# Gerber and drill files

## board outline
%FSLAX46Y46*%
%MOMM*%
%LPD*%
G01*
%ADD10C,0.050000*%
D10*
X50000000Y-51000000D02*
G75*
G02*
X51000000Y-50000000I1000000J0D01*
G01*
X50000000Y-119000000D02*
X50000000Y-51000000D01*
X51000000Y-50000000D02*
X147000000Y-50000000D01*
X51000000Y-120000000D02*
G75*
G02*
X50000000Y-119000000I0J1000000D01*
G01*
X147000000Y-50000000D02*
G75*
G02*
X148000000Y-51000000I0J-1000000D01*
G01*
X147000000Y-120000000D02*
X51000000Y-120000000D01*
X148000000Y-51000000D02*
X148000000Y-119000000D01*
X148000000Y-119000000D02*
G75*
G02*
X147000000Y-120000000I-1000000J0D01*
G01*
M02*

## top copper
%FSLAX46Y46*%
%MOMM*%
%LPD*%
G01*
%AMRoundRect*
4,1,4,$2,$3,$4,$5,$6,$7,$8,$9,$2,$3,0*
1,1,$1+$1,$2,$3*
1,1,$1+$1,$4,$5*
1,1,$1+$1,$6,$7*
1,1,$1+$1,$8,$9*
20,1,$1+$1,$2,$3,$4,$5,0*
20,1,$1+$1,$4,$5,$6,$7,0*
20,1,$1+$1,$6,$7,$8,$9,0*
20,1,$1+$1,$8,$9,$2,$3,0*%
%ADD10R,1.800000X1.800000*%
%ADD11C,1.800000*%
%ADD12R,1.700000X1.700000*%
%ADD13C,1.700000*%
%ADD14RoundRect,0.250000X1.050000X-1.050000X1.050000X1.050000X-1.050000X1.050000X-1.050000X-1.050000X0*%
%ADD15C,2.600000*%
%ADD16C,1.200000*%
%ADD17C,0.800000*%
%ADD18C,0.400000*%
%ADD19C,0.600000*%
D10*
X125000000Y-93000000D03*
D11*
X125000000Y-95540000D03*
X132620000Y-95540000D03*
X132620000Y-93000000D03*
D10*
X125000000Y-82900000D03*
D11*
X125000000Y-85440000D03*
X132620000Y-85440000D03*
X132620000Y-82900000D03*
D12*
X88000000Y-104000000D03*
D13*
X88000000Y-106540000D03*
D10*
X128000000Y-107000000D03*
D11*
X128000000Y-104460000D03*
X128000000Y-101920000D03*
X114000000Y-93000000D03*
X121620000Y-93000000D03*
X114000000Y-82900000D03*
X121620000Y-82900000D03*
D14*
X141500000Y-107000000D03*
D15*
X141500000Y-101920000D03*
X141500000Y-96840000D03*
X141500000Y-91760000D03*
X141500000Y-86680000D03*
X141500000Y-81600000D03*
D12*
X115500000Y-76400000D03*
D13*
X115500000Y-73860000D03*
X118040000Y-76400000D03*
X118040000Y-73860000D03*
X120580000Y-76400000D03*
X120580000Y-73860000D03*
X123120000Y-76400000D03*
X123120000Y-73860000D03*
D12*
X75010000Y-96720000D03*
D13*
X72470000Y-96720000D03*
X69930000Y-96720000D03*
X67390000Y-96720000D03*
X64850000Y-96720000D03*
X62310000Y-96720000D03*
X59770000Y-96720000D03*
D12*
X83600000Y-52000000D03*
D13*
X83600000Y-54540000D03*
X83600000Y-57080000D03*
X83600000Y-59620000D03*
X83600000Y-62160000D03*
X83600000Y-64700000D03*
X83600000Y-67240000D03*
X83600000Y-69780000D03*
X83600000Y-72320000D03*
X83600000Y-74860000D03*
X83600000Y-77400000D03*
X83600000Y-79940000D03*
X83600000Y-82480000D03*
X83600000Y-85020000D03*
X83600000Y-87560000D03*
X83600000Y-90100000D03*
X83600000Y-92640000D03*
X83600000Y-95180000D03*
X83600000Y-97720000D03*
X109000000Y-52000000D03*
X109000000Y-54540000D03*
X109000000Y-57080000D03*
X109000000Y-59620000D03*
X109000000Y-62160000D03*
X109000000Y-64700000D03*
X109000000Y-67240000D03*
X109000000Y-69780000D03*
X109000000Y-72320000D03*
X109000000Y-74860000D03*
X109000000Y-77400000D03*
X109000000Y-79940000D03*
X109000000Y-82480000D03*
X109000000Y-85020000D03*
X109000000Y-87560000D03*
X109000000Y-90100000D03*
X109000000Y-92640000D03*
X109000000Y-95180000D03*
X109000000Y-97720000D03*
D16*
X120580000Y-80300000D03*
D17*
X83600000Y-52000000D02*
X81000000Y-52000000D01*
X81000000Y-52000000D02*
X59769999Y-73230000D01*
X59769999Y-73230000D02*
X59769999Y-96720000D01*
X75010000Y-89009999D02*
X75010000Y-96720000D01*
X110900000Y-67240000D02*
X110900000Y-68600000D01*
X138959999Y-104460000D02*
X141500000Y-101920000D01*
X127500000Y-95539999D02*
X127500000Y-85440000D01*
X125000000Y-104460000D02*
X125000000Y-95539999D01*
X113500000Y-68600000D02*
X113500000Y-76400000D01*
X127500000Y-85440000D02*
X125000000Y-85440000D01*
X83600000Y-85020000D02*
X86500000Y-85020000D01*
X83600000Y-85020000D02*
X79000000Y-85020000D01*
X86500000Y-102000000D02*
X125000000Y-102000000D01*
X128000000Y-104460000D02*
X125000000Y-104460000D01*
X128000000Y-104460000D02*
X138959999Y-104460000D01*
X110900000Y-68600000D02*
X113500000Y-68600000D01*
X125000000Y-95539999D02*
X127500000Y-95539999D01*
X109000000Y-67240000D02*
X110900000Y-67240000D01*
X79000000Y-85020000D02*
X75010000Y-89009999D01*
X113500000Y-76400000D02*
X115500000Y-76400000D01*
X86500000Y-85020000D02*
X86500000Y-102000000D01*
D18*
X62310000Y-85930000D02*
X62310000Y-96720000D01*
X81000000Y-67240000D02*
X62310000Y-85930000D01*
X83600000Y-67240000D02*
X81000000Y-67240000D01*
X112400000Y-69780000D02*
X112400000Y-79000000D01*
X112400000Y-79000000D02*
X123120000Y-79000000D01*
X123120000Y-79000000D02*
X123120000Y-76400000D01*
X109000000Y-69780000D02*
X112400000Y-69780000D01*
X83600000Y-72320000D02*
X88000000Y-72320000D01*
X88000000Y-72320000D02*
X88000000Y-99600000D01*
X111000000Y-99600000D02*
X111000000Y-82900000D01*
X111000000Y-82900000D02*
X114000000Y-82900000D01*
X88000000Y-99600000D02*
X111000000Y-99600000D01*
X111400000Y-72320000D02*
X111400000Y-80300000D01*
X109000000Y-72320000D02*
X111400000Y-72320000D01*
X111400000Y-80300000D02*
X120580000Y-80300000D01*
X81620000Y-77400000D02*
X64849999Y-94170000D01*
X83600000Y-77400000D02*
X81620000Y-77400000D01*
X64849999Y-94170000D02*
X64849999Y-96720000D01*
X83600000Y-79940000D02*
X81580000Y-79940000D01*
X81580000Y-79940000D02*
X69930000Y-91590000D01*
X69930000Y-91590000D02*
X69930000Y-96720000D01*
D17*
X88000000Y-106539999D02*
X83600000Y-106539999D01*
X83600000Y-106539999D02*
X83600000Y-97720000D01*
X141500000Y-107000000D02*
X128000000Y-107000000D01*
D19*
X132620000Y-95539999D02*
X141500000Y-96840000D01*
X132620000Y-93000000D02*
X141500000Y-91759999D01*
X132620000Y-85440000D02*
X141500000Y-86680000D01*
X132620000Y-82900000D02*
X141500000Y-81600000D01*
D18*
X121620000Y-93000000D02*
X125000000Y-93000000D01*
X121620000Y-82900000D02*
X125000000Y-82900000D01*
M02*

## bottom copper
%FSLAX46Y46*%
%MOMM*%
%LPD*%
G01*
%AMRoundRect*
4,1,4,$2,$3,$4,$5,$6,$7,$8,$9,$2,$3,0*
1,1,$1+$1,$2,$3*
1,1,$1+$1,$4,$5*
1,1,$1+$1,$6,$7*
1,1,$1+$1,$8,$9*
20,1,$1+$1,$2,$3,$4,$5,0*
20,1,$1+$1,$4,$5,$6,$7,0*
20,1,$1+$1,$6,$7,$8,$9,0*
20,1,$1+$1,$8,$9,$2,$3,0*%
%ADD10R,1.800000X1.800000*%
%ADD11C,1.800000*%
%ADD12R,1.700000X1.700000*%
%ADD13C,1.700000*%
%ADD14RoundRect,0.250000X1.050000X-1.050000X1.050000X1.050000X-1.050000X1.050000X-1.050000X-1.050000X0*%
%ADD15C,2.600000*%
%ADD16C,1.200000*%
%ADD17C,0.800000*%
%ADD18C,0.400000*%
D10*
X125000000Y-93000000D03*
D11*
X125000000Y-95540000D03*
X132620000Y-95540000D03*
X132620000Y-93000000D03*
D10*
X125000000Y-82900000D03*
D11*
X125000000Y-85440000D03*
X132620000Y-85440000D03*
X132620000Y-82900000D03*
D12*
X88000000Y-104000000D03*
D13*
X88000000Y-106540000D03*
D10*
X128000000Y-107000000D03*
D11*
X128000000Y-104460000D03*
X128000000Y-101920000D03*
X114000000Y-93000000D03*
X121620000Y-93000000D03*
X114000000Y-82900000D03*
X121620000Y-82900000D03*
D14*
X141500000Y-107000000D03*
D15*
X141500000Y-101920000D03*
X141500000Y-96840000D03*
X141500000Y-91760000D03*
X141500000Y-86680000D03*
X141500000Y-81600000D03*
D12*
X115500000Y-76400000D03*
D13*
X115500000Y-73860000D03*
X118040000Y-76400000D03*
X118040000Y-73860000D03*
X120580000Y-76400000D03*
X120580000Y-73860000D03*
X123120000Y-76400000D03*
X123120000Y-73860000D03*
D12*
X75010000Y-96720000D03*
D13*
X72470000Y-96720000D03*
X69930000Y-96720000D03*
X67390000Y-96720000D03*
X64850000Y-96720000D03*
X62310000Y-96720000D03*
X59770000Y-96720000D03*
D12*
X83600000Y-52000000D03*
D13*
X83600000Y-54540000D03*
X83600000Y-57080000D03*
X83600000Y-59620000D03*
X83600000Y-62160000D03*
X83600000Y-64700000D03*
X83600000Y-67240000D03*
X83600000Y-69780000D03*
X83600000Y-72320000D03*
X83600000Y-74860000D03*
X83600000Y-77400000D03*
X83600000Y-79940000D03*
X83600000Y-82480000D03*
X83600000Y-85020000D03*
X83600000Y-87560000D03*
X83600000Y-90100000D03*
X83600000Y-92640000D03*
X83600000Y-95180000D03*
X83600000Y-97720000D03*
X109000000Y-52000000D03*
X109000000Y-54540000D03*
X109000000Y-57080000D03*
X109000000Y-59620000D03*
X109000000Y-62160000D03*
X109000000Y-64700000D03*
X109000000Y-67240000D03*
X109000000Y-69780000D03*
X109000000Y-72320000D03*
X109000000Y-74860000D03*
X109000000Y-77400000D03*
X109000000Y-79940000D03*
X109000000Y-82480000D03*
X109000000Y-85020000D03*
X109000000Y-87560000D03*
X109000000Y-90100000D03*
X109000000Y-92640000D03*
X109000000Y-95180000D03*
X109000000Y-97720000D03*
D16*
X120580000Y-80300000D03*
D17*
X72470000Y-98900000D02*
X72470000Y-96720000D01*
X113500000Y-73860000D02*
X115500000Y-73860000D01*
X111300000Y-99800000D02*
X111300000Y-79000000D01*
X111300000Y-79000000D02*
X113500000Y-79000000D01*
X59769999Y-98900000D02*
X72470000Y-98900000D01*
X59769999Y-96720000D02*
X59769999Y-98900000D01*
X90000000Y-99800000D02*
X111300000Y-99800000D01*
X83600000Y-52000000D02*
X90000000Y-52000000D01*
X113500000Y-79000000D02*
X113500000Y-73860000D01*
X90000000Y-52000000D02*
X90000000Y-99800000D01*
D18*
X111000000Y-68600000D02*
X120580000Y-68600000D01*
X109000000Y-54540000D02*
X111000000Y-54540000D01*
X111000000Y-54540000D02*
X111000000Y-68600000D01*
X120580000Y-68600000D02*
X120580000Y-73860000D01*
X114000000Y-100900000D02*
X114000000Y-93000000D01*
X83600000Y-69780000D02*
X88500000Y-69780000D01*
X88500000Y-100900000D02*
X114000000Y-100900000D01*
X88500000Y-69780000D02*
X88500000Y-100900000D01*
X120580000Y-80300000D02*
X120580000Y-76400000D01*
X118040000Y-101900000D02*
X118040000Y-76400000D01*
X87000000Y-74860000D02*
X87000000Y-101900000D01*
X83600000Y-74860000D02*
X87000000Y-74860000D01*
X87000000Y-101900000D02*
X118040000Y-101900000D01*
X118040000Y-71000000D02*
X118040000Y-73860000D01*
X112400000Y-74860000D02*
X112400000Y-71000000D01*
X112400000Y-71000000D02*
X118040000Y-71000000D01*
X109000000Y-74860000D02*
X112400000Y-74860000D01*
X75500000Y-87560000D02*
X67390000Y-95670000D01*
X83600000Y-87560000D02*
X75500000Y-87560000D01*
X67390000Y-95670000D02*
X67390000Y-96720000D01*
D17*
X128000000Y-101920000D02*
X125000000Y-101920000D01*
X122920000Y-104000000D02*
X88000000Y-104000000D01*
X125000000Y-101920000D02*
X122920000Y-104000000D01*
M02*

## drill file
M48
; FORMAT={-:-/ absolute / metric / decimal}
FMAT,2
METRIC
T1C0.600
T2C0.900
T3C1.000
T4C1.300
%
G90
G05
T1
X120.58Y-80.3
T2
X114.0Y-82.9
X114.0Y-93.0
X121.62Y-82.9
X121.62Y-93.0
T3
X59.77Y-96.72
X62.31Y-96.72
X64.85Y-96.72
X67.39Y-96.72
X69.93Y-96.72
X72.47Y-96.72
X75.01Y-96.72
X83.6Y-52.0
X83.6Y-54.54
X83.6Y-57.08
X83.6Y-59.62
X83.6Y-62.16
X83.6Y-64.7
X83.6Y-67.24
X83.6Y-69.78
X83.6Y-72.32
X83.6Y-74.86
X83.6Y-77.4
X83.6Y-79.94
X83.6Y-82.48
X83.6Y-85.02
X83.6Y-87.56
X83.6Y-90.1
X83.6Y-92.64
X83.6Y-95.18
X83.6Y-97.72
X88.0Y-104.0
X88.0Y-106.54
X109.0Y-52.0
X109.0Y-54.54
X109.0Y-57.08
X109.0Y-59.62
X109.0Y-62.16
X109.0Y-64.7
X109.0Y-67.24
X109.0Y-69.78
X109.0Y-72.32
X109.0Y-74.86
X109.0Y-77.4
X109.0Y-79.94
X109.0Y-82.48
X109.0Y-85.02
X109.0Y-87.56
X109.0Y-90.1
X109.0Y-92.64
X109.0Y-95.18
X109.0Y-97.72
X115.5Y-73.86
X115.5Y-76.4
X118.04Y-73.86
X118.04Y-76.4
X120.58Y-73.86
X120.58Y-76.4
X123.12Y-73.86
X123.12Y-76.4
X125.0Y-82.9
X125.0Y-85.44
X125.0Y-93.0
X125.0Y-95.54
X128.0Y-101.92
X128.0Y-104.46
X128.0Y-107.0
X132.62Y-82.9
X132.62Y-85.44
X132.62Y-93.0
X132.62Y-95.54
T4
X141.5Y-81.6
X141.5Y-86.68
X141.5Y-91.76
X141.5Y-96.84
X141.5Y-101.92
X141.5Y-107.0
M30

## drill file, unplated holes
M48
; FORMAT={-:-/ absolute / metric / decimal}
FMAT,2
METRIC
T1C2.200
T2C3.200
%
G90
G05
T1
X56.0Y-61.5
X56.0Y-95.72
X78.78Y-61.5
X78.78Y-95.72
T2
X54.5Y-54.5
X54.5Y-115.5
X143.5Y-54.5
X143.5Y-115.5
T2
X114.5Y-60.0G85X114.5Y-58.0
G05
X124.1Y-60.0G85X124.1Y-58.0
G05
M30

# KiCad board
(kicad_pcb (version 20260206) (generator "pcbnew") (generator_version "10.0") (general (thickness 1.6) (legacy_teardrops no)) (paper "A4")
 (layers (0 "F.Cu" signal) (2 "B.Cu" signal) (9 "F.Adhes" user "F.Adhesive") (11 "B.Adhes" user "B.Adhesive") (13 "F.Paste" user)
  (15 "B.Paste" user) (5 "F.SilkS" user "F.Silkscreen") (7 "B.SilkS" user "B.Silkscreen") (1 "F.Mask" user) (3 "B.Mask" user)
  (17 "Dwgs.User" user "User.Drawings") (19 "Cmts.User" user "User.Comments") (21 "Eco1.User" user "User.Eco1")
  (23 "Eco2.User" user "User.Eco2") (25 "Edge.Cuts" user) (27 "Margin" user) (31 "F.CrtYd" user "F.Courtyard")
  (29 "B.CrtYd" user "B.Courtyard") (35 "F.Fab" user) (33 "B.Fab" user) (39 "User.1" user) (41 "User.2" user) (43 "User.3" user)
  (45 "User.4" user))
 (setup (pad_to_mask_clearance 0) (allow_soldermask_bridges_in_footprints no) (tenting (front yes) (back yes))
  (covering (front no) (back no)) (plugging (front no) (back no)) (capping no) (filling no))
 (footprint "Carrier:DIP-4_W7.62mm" (layer "F.Cu") (at 125 93)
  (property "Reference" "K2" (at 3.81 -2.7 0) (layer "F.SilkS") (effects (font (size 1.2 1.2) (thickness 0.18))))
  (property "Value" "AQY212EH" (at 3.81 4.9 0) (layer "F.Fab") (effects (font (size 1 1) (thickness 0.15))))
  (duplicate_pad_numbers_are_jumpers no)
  (pad "1" thru_hole rect (at 0 0) (size 1.8 1.8) (drill 1) (layers "*.Cu" "*.Mask") (remove_unused_layers no) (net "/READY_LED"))
  (pad "2" thru_hole circle (at 0 2.54) (size 1.8 1.8) (drill 1) (layers "*.Cu" "*.Mask") (remove_unused_layers no) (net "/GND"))
  (pad "3" thru_hole circle (at 7.62 2.54) (size 1.8 1.8) (drill 1) (layers "*.Cu" "*.Mask") (remove_unused_layers no) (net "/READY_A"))
  (pad "4" thru_hole circle (at 7.62 0) (size 1.8 1.8) (drill 1) (layers "*.Cu" "*.Mask") (remove_unused_layers no) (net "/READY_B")))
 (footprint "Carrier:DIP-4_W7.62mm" (layer "F.Cu") (at 125 82.9)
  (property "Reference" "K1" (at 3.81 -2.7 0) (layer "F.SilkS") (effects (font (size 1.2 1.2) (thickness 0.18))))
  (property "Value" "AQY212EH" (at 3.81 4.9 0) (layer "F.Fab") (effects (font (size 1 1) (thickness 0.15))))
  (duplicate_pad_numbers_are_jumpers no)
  (pad "1" thru_hole rect (at 0 0) (size 1.8 1.8) (drill 1) (layers "*.Cu" "*.Mask") (remove_unused_layers no) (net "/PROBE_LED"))
  (pad "2" thru_hole circle (at 0 2.54) (size 1.8 1.8) (drill 1) (layers "*.Cu" "*.Mask") (remove_unused_layers no) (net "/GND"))
  (pad "3" thru_hole circle (at 7.62 2.54) (size 1.8 1.8) (drill 1) (layers "*.Cu" "*.Mask") (remove_unused_layers no) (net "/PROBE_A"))
  (pad "4" thru_hole circle (at 7.62 0) (size 1.8 1.8) (drill 1) (layers "*.Cu" "*.Mask") (remove_unused_layers no) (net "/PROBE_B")))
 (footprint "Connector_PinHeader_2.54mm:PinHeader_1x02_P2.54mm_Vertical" (layer "F.Cu") (at 88 104)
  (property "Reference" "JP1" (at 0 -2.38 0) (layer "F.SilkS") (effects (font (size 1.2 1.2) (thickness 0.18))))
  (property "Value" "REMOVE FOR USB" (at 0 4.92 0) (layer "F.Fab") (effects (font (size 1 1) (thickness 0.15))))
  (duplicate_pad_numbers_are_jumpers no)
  (pad "1" thru_hole rect (at 0 0) (size 1.7 1.7) (drill 1) (layers "*.Cu" "*.Mask") (remove_unused_layers no) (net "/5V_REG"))
  (pad "2" thru_hole circle (at 0 2.54) (size 1.7 1.7) (drill 1) (layers "*.Cu" "*.Mask") (remove_unused_layers no) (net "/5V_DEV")))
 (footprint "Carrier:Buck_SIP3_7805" (layer "F.Cu") (at 128 107 90)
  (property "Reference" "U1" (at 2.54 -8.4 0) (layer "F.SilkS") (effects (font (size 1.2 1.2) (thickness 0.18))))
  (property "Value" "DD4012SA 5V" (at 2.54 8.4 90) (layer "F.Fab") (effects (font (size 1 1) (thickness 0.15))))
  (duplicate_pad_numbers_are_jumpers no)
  (pad "1" thru_hole rect (at 0 0 90) (size 1.8 1.8) (drill 1) (layers "*.Cu" "*.Mask") (remove_unused_layers no) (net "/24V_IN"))
  (pad "2" thru_hole circle (at 2.54 0 90) (size 1.8 1.8) (drill 1) (layers "*.Cu" "*.Mask") (remove_unused_layers no) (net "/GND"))
  (pad "3" thru_hole circle (at 5.08 0 90) (size 1.8 1.8) (drill 1) (layers "*.Cu" "*.Mask") (remove_unused_layers no) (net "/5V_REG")))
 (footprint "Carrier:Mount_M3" (layer "F.Cu") (at 54.5 54.5)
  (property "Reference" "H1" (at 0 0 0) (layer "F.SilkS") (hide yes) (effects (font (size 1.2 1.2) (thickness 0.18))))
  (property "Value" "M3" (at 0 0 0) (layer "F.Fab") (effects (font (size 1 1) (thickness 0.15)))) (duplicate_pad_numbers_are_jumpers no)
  (pad "" np_thru_hole circle (at 0 0) (size 3.2 3.2) (drill 3.2) (layers "*.Cu" "*.Mask"))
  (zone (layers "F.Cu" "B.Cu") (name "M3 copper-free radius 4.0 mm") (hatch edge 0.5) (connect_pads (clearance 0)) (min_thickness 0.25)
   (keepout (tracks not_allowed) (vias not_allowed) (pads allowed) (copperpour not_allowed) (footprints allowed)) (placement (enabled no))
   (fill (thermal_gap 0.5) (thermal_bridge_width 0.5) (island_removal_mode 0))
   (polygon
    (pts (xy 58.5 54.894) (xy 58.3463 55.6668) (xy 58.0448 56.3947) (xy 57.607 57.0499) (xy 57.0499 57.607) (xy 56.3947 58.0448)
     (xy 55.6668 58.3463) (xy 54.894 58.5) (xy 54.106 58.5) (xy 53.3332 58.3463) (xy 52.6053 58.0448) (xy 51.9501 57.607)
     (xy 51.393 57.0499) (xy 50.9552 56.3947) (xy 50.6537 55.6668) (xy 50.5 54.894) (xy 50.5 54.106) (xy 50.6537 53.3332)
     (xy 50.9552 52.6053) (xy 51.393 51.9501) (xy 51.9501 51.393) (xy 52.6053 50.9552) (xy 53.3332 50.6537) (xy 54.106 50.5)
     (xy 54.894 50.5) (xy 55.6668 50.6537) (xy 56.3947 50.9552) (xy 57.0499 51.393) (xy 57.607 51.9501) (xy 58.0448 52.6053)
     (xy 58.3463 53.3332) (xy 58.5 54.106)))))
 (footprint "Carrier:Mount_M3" (layer "F.Cu") (at 143.5 54.5)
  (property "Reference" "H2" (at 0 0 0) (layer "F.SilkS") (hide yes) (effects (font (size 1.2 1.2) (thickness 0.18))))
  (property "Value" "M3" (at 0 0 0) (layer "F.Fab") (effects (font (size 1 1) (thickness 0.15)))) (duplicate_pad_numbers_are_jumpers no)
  (pad "" np_thru_hole circle (at 0 0) (size 3.2 3.2) (drill 3.2) (layers "*.Cu" "*.Mask"))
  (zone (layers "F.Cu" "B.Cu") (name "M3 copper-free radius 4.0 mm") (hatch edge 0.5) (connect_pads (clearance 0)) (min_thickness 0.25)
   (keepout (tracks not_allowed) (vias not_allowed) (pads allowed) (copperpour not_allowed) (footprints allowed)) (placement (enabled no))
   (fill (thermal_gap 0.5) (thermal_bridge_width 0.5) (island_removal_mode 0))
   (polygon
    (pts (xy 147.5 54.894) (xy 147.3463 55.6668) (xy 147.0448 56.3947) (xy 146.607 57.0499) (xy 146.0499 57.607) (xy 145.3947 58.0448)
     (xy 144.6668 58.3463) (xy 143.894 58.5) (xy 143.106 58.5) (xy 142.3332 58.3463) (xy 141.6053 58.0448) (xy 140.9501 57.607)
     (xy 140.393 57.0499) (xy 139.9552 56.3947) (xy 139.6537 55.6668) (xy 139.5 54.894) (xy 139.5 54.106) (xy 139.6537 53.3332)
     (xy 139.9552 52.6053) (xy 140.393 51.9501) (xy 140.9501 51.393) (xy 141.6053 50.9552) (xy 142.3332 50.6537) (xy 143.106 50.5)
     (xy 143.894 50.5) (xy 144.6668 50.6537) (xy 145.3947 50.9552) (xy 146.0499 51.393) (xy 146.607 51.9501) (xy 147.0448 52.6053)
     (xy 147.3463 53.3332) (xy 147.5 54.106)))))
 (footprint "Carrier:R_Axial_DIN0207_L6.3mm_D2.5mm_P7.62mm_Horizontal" (layer "F.Cu") (at 114 93)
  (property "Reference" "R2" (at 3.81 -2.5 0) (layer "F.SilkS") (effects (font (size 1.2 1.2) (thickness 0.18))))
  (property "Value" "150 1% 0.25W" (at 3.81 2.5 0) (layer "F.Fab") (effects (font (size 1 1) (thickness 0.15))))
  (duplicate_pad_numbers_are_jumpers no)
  (pad "1" thru_hole circle (at 0 0) (size 1.8 1.8) (drill 0.9) (layers "*.Cu" "*.Mask") (remove_unused_layers no) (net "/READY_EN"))
  (pad "2" thru_hole circle (at 7.62 0) (size 1.8 1.8) (drill 0.9) (layers "*.Cu" "*.Mask") (remove_unused_layers no) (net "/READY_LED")))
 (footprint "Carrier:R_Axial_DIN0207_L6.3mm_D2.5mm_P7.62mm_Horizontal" (layer "F.Cu") (at 114 82.9)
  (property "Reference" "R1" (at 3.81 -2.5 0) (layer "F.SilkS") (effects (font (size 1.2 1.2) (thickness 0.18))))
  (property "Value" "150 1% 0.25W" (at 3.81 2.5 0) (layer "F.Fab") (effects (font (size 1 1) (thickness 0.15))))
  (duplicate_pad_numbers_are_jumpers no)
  (pad "1" thru_hole circle (at 0 0) (size 1.8 1.8) (drill 0.9) (layers "*.Cu" "*.Mask") (remove_unused_layers no) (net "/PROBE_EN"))
  (pad "2" thru_hole circle (at 7.62 0) (size 1.8 1.8) (drill 0.9) (layers "*.Cu" "*.Mask") (remove_unused_layers no) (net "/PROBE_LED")))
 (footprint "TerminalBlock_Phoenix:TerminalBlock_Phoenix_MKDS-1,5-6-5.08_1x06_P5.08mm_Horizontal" (layer "F.Cu") (at 141.5 107 90)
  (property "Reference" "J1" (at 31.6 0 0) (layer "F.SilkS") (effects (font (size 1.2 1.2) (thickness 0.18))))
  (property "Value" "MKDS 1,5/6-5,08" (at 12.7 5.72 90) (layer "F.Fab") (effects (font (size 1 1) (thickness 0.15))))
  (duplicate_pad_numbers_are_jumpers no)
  (pad "1" thru_hole roundrect (at 0 0 90) (size 2.6 2.6) (drill 1.3) (layers "*.Cu" "*.Mask") (remove_unused_layers no)
   (roundrect_rratio 0.096154) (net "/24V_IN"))
  (pad "2" thru_hole circle (at 5.08 0 90) (size 2.6 2.6) (drill 1.3) (layers "*.Cu" "*.Mask") (remove_unused_layers no) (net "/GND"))
  (pad "3" thru_hole circle (at 10.16 0 90) (size 2.6 2.6) (drill 1.3) (layers "*.Cu" "*.Mask") (remove_unused_layers no) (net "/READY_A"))
  (pad "4" thru_hole circle (at 15.24 0 90) (size 2.6 2.6) (drill 1.3) (layers "*.Cu" "*.Mask") (remove_unused_layers no) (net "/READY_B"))
  (pad "5" thru_hole circle (at 20.32 0 90) (size 2.6 2.6) (drill 1.3) (layers "*.Cu" "*.Mask") (remove_unused_layers no) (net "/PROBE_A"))
  (pad "6" thru_hole circle (at 25.4 0 90) (size 2.6 2.6) (drill 1.3) (layers "*.Cu" "*.Mask") (remove_unused_layers no) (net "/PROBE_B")))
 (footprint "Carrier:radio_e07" (layer "F.Cu") (at 115.5 76.4 180)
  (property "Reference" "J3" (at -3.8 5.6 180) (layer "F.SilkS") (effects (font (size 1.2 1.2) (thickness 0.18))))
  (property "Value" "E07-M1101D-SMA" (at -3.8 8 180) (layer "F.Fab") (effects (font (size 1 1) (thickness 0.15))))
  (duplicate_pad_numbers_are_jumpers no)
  (pad "" np_thru_hole oval (at -8.6 17.4 180) (size 3.2 5.2) (drill oval 3.2 5.2) (layers "*.Cu" "*.Mask"))
  (pad "" np_thru_hole oval (at 1 17.4 180) (size 3.2 5.2) (drill oval 3.2 5.2) (layers "*.Cu" "*.Mask"))
  (pad "1" thru_hole rect (at 0 0 180) (size 1.7 1.7) (drill 1) (layers "*.Cu" "*.Mask") (remove_unused_layers no) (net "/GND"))
  (pad "2" thru_hole circle (at 0 2.54 180) (size 1.7 1.7) (drill 1) (layers "*.Cu" "*.Mask") (remove_unused_layers no) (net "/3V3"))
  (pad "3" thru_hole circle (at -2.54 0 180) (size 1.7 1.7) (drill 1) (layers "*.Cu" "*.Mask") (remove_unused_layers no) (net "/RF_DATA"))
  (pad "4" thru_hole circle (at -2.54 2.54 180) (size 1.7 1.7) (drill 1) (layers "*.Cu" "*.Mask") (remove_unused_layers no) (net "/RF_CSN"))
  (pad "5" thru_hole circle (at -5.08 0 180) (size 1.7 1.7) (drill 1) (layers "*.Cu" "*.Mask") (remove_unused_layers no) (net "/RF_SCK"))
  (pad "6" thru_hole circle (at -5.08 2.54 180) (size 1.7 1.7) (drill 1) (layers "*.Cu" "*.Mask") (remove_unused_layers no) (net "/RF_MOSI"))
  (pad "7" thru_hole circle (at -7.62 0 180) (size 1.7 1.7) (drill 1) (layers "*.Cu" "*.Mask") (remove_unused_layers no) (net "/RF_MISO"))
  (pad "8" thru_hole circle (at -7.62 2.54 180) (size 1.7 1.7) (drill 1) (layers "*.Cu" "*.Mask") (remove_unused_layers no)
   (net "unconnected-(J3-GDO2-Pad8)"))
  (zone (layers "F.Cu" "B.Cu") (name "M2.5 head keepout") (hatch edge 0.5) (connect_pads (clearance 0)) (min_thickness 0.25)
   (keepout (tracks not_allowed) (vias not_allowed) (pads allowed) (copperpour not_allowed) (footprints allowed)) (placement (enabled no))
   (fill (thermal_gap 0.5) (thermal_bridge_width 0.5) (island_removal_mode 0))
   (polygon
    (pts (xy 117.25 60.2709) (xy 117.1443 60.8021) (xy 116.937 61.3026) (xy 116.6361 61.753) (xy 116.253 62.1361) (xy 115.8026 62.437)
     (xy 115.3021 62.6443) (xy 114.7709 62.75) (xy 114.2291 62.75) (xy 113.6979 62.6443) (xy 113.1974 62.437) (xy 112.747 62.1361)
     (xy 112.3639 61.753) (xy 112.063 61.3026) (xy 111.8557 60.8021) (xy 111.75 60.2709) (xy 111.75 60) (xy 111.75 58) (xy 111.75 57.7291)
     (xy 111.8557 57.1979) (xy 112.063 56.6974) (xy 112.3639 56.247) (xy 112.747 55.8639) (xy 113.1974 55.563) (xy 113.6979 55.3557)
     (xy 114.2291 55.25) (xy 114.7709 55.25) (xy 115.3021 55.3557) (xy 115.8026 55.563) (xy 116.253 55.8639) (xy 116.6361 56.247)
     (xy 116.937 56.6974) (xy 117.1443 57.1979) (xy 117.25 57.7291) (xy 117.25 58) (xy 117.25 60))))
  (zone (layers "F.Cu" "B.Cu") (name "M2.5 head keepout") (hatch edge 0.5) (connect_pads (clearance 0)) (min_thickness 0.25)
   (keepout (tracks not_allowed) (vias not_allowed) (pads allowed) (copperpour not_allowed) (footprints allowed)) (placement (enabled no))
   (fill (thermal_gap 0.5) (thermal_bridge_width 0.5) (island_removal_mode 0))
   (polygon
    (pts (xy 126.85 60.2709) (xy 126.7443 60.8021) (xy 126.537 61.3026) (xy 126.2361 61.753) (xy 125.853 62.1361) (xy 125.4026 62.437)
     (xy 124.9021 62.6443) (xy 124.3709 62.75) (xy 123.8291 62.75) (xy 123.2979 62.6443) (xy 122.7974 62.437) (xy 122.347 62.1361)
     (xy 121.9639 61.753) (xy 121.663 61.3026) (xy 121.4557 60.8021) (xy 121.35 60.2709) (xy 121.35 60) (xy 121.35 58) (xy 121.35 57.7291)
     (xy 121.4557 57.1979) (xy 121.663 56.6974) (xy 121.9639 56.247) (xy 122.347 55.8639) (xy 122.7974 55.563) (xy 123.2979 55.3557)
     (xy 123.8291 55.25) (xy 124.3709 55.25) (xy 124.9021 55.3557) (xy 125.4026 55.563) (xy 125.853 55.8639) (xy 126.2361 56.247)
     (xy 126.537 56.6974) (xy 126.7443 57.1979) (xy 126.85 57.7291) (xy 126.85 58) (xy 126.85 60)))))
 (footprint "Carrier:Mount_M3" (layer "F.Cu") (at 143.5 115.5)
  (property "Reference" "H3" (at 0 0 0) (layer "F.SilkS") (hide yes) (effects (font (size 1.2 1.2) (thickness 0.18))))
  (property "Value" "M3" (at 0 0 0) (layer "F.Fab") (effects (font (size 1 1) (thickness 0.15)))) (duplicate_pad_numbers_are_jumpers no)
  (pad "" np_thru_hole circle (at 0 0) (size 3.2 3.2) (drill 3.2) (layers "*.Cu" "*.Mask"))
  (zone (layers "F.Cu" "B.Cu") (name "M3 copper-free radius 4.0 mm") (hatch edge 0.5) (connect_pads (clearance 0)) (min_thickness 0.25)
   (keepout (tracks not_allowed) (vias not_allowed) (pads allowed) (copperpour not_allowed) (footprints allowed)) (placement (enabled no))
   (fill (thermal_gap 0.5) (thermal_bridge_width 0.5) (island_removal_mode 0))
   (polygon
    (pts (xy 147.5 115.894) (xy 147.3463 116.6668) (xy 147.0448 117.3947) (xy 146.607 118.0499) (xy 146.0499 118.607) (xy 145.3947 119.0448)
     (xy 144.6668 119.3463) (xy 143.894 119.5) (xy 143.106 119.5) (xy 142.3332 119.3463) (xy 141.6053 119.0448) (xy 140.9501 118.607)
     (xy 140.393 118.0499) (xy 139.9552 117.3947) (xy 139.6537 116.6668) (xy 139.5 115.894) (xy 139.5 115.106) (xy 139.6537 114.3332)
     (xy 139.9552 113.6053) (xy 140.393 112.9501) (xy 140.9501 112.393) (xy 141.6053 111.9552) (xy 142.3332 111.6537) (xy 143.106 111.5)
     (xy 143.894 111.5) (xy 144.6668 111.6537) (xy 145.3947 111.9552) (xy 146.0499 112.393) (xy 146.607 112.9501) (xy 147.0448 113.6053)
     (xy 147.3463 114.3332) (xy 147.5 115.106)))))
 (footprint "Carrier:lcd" (layer "F.Cu") (at 67.39 78.94 180)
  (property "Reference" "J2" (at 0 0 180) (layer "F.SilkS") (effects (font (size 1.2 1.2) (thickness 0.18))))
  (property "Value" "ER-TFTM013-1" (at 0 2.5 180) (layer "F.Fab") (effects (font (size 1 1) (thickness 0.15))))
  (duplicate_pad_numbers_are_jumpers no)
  (pad "" np_thru_hole circle (at -11.39 -16.78 180) (size 2.2 2.2) (drill 2.2) (layers "*.Cu" "*.Mask"))
  (pad "" np_thru_hole circle (at -11.39 17.44 180) (size 2.2 2.2) (drill 2.2) (layers "*.Cu" "*.Mask"))
  (pad "" np_thru_hole circle (at 11.39 -16.78 180) (size 2.2 2.2) (drill 2.2) (layers "*.Cu" "*.Mask"))
  (pad "" np_thru_hole circle (at 11.39 17.44 180) (size 2.2 2.2) (drill 2.2) (layers "*.Cu" "*.Mask"))
  (pad "1" thru_hole rect (at -7.62 -17.78 180) (size 1.7 1.7) (drill 1) (layers "*.Cu" "*.Mask") (remove_unused_layers no) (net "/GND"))
  (pad "2" thru_hole circle (at -5.08 -17.78 180) (size 1.7 1.7) (drill 1) (layers "*.Cu" "*.Mask") (remove_unused_layers no) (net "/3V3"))
  (pad "3" thru_hole circle (at -2.54 -17.78 180) (size 1.7 1.7) (drill 1) (layers "*.Cu" "*.Mask") (remove_unused_layers no)
   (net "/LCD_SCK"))
  (pad "4" thru_hole circle (at 0 -17.78 180) (size 1.7 1.7) (drill 1) (layers "*.Cu" "*.Mask") (remove_unused_layers no) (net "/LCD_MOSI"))
  (pad "5" thru_hole circle (at 2.54 -17.78 180) (size 1.7 1.7) (drill 1) (layers "*.Cu" "*.Mask") (remove_unused_layers no)
   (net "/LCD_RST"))
  (pad "6" thru_hole circle (at 5.08 -17.78 180) (size 1.7 1.7) (drill 1) (layers "*.Cu" "*.Mask") (remove_unused_layers no) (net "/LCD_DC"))
  (pad "7" thru_hole circle (at 7.62 -17.78 180) (size 1.7 1.7) (drill 1) (layers "*.Cu" "*.Mask") (remove_unused_layers no) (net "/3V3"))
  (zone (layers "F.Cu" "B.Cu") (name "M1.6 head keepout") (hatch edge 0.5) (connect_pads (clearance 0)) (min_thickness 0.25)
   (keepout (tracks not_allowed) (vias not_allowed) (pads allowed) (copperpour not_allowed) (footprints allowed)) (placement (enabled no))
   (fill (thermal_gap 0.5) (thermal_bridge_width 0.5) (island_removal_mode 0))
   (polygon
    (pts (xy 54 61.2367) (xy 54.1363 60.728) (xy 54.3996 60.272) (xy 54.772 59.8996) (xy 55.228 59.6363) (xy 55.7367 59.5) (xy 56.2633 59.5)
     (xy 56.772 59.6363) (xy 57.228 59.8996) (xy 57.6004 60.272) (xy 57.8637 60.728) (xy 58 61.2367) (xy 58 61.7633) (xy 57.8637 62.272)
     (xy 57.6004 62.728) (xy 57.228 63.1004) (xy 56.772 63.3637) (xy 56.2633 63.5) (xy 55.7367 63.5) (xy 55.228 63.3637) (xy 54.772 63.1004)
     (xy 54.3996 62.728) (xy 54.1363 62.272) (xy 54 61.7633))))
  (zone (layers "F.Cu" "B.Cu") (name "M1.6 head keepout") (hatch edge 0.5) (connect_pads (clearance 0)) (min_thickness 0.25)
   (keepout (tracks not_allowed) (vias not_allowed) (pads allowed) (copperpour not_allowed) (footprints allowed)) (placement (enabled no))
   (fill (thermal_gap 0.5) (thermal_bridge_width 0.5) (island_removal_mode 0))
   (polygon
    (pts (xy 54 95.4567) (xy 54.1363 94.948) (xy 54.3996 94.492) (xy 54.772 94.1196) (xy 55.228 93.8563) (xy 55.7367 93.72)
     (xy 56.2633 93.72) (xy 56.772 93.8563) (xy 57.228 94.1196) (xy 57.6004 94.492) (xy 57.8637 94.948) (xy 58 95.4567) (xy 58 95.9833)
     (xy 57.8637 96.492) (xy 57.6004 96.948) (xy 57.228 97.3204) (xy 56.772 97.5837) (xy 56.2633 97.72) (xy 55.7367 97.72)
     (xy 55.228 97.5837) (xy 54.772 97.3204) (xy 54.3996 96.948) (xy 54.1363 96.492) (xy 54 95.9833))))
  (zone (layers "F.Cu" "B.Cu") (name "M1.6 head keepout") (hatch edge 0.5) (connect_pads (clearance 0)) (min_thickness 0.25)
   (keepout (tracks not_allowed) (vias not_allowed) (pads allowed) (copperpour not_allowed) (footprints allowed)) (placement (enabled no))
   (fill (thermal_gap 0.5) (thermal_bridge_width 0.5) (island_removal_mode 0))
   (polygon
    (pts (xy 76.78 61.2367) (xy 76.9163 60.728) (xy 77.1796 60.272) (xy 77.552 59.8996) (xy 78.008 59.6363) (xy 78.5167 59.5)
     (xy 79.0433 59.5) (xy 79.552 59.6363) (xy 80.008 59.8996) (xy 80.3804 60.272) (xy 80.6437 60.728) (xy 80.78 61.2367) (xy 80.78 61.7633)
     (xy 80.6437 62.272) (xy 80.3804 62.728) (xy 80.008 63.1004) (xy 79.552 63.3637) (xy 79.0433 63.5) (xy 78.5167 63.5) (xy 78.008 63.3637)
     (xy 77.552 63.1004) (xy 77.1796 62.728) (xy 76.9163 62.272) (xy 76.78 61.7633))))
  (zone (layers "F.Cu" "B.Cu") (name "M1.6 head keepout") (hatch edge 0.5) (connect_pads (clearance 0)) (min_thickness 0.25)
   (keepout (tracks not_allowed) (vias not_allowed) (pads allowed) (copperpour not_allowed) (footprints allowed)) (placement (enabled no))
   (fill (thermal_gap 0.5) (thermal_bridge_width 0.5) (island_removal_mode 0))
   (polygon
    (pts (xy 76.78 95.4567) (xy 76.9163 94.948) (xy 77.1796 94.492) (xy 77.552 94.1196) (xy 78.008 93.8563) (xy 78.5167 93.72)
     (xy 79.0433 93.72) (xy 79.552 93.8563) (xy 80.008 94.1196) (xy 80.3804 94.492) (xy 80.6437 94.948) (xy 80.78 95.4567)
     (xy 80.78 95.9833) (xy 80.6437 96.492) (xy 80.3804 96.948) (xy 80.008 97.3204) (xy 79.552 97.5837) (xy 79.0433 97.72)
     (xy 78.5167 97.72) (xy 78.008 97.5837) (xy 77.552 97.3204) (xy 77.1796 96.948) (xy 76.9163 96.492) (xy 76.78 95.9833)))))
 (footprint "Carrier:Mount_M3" (layer "F.Cu") (at 54.5 115.5)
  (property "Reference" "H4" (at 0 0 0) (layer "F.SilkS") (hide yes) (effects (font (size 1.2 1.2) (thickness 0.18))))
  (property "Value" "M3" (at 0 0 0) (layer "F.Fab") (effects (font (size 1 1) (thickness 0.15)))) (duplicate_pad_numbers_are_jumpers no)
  (pad "" np_thru_hole circle (at 0 0) (size 3.2 3.2) (drill 3.2) (layers "*.Cu" "*.Mask"))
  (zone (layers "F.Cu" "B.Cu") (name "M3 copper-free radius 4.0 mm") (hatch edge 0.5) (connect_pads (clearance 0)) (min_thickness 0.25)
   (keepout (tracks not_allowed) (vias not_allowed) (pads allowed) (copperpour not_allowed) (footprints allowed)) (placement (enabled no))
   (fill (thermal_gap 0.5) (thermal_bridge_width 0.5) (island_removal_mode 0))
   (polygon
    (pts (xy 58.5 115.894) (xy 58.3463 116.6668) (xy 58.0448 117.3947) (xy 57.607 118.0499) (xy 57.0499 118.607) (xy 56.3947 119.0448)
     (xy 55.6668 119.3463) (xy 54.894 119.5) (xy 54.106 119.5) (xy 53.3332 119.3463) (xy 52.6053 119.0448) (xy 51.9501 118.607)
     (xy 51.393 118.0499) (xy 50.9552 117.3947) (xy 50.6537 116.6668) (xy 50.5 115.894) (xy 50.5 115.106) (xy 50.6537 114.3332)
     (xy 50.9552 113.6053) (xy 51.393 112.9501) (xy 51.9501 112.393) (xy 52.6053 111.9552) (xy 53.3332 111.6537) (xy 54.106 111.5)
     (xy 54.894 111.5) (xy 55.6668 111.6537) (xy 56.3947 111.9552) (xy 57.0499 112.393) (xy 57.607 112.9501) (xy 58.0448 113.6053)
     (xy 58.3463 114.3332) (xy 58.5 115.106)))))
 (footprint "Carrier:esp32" (layer "F.Cu") (at 96.3 52)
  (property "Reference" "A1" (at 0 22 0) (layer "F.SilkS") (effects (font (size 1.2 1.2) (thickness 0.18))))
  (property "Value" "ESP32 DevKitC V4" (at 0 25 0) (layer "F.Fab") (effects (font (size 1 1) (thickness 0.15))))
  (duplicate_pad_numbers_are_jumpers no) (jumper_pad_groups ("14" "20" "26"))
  (pad "1" thru_hole rect (at -12.7 0) (size 1.7 1.7) (drill 1) (layers "*.Cu" "*.Mask") (remove_unused_layers no) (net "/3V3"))
  (pad "2" thru_hole circle (at -12.7 2.54) (size 1.7 1.7) (drill 1) (layers "*.Cu" "*.Mask") (remove_unused_layers no)
   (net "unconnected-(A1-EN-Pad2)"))
  (pad "3" thru_hole circle (at -12.7 5.08) (size 1.7 1.7) (drill 1) (layers "*.Cu" "*.Mask") (remove_unused_layers no)
   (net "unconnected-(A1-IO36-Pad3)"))
  (pad "4" thru_hole circle (at -12.7 7.62) (size 1.7 1.7) (drill 1) (layers "*.Cu" "*.Mask") (remove_unused_layers no)
   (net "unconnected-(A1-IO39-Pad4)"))
  (pad "5" thru_hole circle (at -12.7 10.16) (size 1.7 1.7) (drill 1) (layers "*.Cu" "*.Mask") (remove_unused_layers no)
   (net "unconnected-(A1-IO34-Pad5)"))
  (pad "6" thru_hole circle (at -12.7 12.7) (size 1.7 1.7) (drill 1) (layers "*.Cu" "*.Mask") (remove_unused_layers no)
   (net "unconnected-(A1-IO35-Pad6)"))
  (pad "7" thru_hole circle (at -12.7 15.24) (size 1.7 1.7) (drill 1) (layers "*.Cu" "*.Mask") (remove_unused_layers no) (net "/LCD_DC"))
  (pad "8" thru_hole circle (at -12.7 17.78) (size 1.7 1.7) (drill 1) (layers "*.Cu" "*.Mask") (remove_unused_layers no) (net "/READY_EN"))
  (pad "9" thru_hole circle (at -12.7 20.32) (size 1.7 1.7) (drill 1) (layers "*.Cu" "*.Mask") (remove_unused_layers no) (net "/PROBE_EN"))
  (pad "10" thru_hole circle (at -12.7 22.86) (size 1.7 1.7) (drill 1) (layers "*.Cu" "*.Mask") (remove_unused_layers no) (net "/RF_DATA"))
  (pad "11" thru_hole circle (at -12.7 25.4) (size 1.7 1.7) (drill 1) (layers "*.Cu" "*.Mask") (remove_unused_layers no) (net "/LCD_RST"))
  (pad "12" thru_hole circle (at -12.7 27.94) (size 1.7 1.7) (drill 1) (layers "*.Cu" "*.Mask") (remove_unused_layers no) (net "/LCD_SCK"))
  (pad "13" thru_hole circle (at -12.7 30.48) (size 1.7 1.7) (drill 1) (layers "*.Cu" "*.Mask") (remove_unused_layers no)
   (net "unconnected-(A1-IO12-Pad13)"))
  (pad "14" thru_hole circle (at -12.7 33.02) (size 1.7 1.7) (drill 1) (layers "*.Cu" "*.Mask") (remove_unused_layers no) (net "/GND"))
  (pad "15" thru_hole circle (at -12.7 35.56) (size 1.7 1.7) (drill 1) (layers "*.Cu" "*.Mask") (remove_unused_layers no) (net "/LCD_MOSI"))
  (pad "16" thru_hole circle (at -12.7 38.1) (size 1.7 1.7) (drill 1) (layers "*.Cu" "*.Mask") (remove_unused_layers no)
   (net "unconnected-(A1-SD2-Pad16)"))
  (pad "17" thru_hole circle (at -12.7 40.64) (size 1.7 1.7) (drill 1) (layers "*.Cu" "*.Mask") (remove_unused_layers no)
   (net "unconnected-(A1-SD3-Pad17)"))
  (pad "18" thru_hole circle (at -12.7 43.18) (size 1.7 1.7) (drill 1) (layers "*.Cu" "*.Mask") (remove_unused_layers no)
   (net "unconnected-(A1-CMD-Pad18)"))
  (pad "19" thru_hole circle (at -12.7 45.72) (size 1.7 1.7) (drill 1) (layers "*.Cu" "*.Mask") (remove_unused_layers no) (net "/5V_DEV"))
  (pad "20" thru_hole circle (at 12.7 0) (size 1.7 1.7) (drill 1) (layers "*.Cu" "*.Mask") (remove_unused_layers no) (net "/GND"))
  (pad "21" thru_hole circle (at 12.7 2.54) (size 1.7 1.7) (drill 1) (layers "*.Cu" "*.Mask") (remove_unused_layers no) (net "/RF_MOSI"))
  (pad "22" thru_hole circle (at 12.7 5.08) (size 1.7 1.7) (drill 1) (layers "*.Cu" "*.Mask") (remove_unused_layers no)
   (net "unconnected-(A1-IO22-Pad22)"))
  (pad "23" thru_hole circle (at 12.7 7.62) (size 1.7 1.7) (drill 1) (layers "*.Cu" "*.Mask") (remove_unused_layers no)
   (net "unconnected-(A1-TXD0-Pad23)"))
  (pad "24" thru_hole circle (at 12.7 10.16) (size 1.7 1.7) (drill 1) (layers "*.Cu" "*.Mask") (remove_unused_layers no)
   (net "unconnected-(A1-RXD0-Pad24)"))
  (pad "25" thru_hole circle (at 12.7 12.7) (size 1.7 1.7) (drill 1) (layers "*.Cu" "*.Mask") (remove_unused_layers no)
   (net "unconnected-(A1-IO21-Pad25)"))
  (pad "26" thru_hole circle (at 12.7 15.24) (size 1.7 1.7) (drill 1) (layers "*.Cu" "*.Mask") (remove_unused_layers no) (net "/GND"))
  (pad "27" thru_hole circle (at 12.7 17.78) (size 1.7 1.7) (drill 1) (layers "*.Cu" "*.Mask") (remove_unused_layers no) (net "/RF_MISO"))
  (pad "28" thru_hole circle (at 12.7 20.32) (size 1.7 1.7) (drill 1) (layers "*.Cu" "*.Mask") (remove_unused_layers no) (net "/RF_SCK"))
  (pad "29" thru_hole circle (at 12.7 22.86) (size 1.7 1.7) (drill 1) (layers "*.Cu" "*.Mask") (remove_unused_layers no) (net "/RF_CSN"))
  (pad "30" thru_hole circle (at 12.7 25.4) (size 1.7 1.7) (drill 1) (layers "*.Cu" "*.Mask") (remove_unused_layers no)
   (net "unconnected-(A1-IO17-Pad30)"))
  (pad "31" thru_hole circle (at 12.7 27.94) (size 1.7 1.7) (drill 1) (layers "*.Cu" "*.Mask") (remove_unused_layers no)
   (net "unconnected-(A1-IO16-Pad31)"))
  (pad "32" thru_hole circle (at 12.7 30.48) (size 1.7 1.7) (drill 1) (layers "*.Cu" "*.Mask") (remove_unused_layers no)
   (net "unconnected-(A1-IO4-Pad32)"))
  (pad "33" thru_hole circle (at 12.7 33.02) (size 1.7 1.7) (drill 1) (layers "*.Cu" "*.Mask") (remove_unused_layers no)
   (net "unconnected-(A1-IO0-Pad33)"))
  (pad "34" thru_hole circle (at 12.7 35.56) (size 1.7 1.7) (drill 1) (layers "*.Cu" "*.Mask") (remove_unused_layers no)
   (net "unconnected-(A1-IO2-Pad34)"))
  (pad "35" thru_hole circle (at 12.7 38.1) (size 1.7 1.7) (drill 1) (layers "*.Cu" "*.Mask") (remove_unused_layers no)
   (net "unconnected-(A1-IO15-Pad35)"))
  (pad "36" thru_hole circle (at 12.7 40.64) (size 1.7 1.7) (drill 1) (layers "*.Cu" "*.Mask") (remove_unused_layers no)
   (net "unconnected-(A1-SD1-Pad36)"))
  (pad "37" thru_hole circle (at 12.7 43.18) (size 1.7 1.7) (drill 1) (layers "*.Cu" "*.Mask") (remove_unused_layers no)
   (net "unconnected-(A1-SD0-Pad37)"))
  (pad "38" thru_hole circle (at 12.7 45.72) (size 1.7 1.7) (drill 1) (layers "*.Cu" "*.Mask") (remove_unused_layers no)
   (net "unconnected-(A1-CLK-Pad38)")))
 (gr_arc (start 50 51) (mid 50.292893 50.292893) (end 51 50) (stroke (width 0.05) (type default)) (layer "Edge.Cuts"))
 (gr_line (start 50 119) (end 50 51) (stroke (width 0.05) (type default)) (layer "Edge.Cuts"))
 (gr_line (start 51 50) (end 147 50) (stroke (width 0.05) (type default)) (layer "Edge.Cuts"))
 (gr_arc (start 51 120) (mid 50.292893 119.707106) (end 50 119) (stroke (width 0.05) (type default)) (layer "Edge.Cuts"))
 (gr_arc (start 147 50) (mid 147.707106 50.292893) (end 148 51) (stroke (width 0.05) (type default)) (layer "Edge.Cuts"))
 (gr_line (start 147 120) (end 51 120) (stroke (width 0.05) (type default)) (layer "Edge.Cuts"))
 (gr_line (start 148 51) (end 148 119) (stroke (width 0.05) (type default)) (layer "Edge.Cuts"))
 (gr_arc (start 148 119) (mid 147.707106 119.707106) (end 147 120) (stroke (width 0.05) (type default)) (layer "Edge.Cuts"))
 (segment (start 83.6 52) (end 81 52) (width 0.8) (layer "F.Cu") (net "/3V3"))
 (segment (start 81 52) (end 59.769999 73.23) (width 0.8) (layer "F.Cu") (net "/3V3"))
 (segment (start 59.769999 73.23) (end 59.769999 96.72) (width 0.8) (layer "F.Cu") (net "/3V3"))
 (segment (start 72.47 98.9) (end 72.47 96.72) (width 0.8) (layer "B.Cu") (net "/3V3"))
 (segment (start 113.5 73.86) (end 115.5 73.86) (width 0.8) (layer "B.Cu") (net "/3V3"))
 (segment (start 111.3 99.8) (end 111.3 79) (width 0.8) (layer "B.Cu") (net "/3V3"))
 (segment (start 111.3 79) (end 113.5 79) (width 0.8) (layer "B.Cu") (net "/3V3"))
 (segment (start 59.769999 98.9) (end 72.47 98.9) (width 0.8) (layer "B.Cu") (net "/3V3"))
 (segment (start 59.769999 96.72) (end 59.769999 98.9) (width 0.8) (layer "B.Cu") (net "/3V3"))
 (segment (start 90 99.8) (end 111.3 99.8) (width 0.8) (layer "B.Cu") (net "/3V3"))
 (segment (start 83.6 52) (end 90 52) (width 0.8) (layer "B.Cu") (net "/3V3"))
 (segment (start 113.5 79) (end 113.5 73.86) (width 0.8) (layer "B.Cu") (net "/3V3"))
 (segment (start 90 52) (end 90 99.8) (width 0.8) (layer "B.Cu") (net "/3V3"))
 (segment (start 75.01 89.009999) (end 75.01 96.72) (width 0.8) (layer "F.Cu") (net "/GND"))
 (segment (start 110.9 67.24) (end 110.9 68.6) (width 0.8) (layer "F.Cu") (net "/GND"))
 (segment (start 138.959999 104.46) (end 141.5 101.92) (width 0.8) (layer "F.Cu") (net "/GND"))
 (segment (start 127.5 95.539999) (end 127.5 85.44) (width 0.8) (layer "F.Cu") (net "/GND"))
 (segment (start 125 104.46) (end 125 95.539999) (width 0.8) (layer "F.Cu") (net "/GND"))
 (segment (start 113.5 68.6) (end 113.5 76.4) (width 0.8) (layer "F.Cu") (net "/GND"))
 (segment (start 127.5 85.44) (end 125 85.44) (width 0.8) (layer "F.Cu") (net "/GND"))
 (segment (start 83.6 85.02) (end 86.5 85.02) (width 0.8) (layer "F.Cu") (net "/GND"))
 (segment (start 83.6 85.02) (end 79 85.02) (width 0.8) (layer "F.Cu") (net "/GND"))
 (segment (start 86.5 102) (end 125 102) (width 0.8) (layer "F.Cu") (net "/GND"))
 (segment (start 128 104.46) (end 125 104.46) (width 0.8) (layer "F.Cu") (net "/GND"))
 (segment (start 128 104.46) (end 138.959999 104.46) (width 0.8) (layer "F.Cu") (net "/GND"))
 (segment (start 110.9 68.6) (end 113.5 68.6) (width 0.8) (layer "F.Cu") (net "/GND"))
 (segment (start 125 95.539999) (end 127.5 95.539999) (width 0.8) (layer "F.Cu") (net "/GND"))
 (segment (start 109 67.24) (end 110.9 67.24) (width 0.8) (layer "F.Cu") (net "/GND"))
 (segment (start 79 85.02) (end 75.01 89.009999) (width 0.8) (layer "F.Cu") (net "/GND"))
 (segment (start 113.5 76.4) (end 115.5 76.4) (width 0.8) (layer "F.Cu") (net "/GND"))
 (segment (start 86.5 85.02) (end 86.5 102) (width 0.8) (layer "F.Cu") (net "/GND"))
 (segment (start 111 68.6) (end 120.58 68.6) (width 0.4) (layer "B.Cu") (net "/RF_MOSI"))
 (segment (start 109 54.54) (end 111 54.54) (width 0.4) (layer "B.Cu") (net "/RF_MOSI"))
 (segment (start 111 54.54) (end 111 68.6) (width 0.4) (layer "B.Cu") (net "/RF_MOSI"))
 (segment (start 120.58 68.6) (end 120.58 73.86) (width 0.4) (layer "B.Cu") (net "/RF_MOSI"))
 (segment (start 62.31 85.93) (end 62.31 96.72) (width 0.4) (layer "F.Cu") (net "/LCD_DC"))
 (segment (start 81 67.24) (end 62.31 85.93) (width 0.4) (layer "F.Cu") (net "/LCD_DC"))
 (segment (start 83.6 67.24) (end 81 67.24) (width 0.4) (layer "F.Cu") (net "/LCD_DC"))
 (segment (start 114 100.9) (end 114 93) (width 0.4) (layer "B.Cu") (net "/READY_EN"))
 (segment (start 83.6 69.78) (end 88.5 69.78) (width 0.4) (layer "B.Cu") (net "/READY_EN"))
 (segment (start 88.5 100.9) (end 114 100.9) (width 0.4) (layer "B.Cu") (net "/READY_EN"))
 (segment (start 88.5 69.78) (end 88.5 100.9) (width 0.4) (layer "B.Cu") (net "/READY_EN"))
 (segment (start 112.4 69.78) (end 112.4 79) (width 0.4) (layer "F.Cu") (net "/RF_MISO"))
 (segment (start 112.4 79) (end 123.12 79) (width 0.4) (layer "F.Cu") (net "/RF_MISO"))
 (segment (start 123.12 79) (end 123.12 76.4) (width 0.4) (layer "F.Cu") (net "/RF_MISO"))
 (segment (start 109 69.78) (end 112.4 69.78) (width 0.4) (layer "F.Cu") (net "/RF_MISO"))
 (segment (start 83.6 72.32) (end 88 72.32) (width 0.4) (layer "F.Cu") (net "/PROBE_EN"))
 (segment (start 88 72.32) (end 88 99.6) (width 0.4) (layer "F.Cu") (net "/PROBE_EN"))
 (segment (start 111 99.6) (end 111 82.9) (width 0.4) (layer "F.Cu") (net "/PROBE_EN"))
 (segment (start 111 82.9) (end 114 82.9) (width 0.4) (layer "F.Cu") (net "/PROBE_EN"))
 (segment (start 88 99.6) (end 111 99.6) (width 0.4) (layer "F.Cu") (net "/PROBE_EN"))
 (segment (start 111.4 72.32) (end 111.4 80.3) (width 0.4) (layer "F.Cu") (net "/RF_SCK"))
 (segment (start 109 72.32) (end 111.4 72.32) (width 0.4) (layer "F.Cu") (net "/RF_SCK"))
 (segment (start 111.4 80.3) (end 120.58 80.3) (width 0.4) (layer "F.Cu") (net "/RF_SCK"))
 (via (at 120.58 80.3) (size 1.2) (drill 0.6) (layers "F.Cu" "B.Cu") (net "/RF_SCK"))
 (segment (start 120.58 80.3) (end 120.58 76.4) (width 0.4) (layer "B.Cu") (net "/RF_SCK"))
 (segment (start 118.04 101.9) (end 118.04 76.4) (width 0.4) (layer "B.Cu") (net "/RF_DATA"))
 (segment (start 87 74.86) (end 87 101.9) (width 0.4) (layer "B.Cu") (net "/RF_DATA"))
 (segment (start 83.6 74.86) (end 87 74.86) (width 0.4) (layer "B.Cu") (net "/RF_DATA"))
 (segment (start 87 101.9) (end 118.04 101.9) (width 0.4) (layer "B.Cu") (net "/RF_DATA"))
 (segment (start 118.04 71) (end 118.04 73.86) (width 0.4) (layer "B.Cu") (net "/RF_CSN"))
 (segment (start 112.4 74.86) (end 112.4 71) (width 0.4) (layer "B.Cu") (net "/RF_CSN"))
 (segment (start 112.4 71) (end 118.04 71) (width 0.4) (layer "B.Cu") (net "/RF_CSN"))
 (segment (start 109 74.86) (end 112.4 74.86) (width 0.4) (layer "B.Cu") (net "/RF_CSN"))
 (segment (start 81.62 77.4) (end 64.849999 94.17) (width 0.4) (layer "F.Cu") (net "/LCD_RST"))
 (segment (start 83.6 77.4) (end 81.62 77.4) (width 0.4) (layer "F.Cu") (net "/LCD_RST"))
 (segment (start 64.849999 94.17) (end 64.849999 96.72) (width 0.4) (layer "F.Cu") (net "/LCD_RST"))
 (segment (start 83.6 79.94) (end 81.58 79.94) (width 0.4) (layer "F.Cu") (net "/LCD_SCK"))
 (segment (start 81.58 79.94) (end 69.93 91.59) (width 0.4) (layer "F.Cu") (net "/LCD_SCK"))
 (segment (start 69.93 91.59) (end 69.93 96.72) (width 0.4) (layer "F.Cu") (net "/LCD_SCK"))
 (segment (start 75.5 87.56) (end 67.39 95.67) (width 0.4) (layer "B.Cu") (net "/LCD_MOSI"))
 (segment (start 83.6 87.56) (end 75.5 87.56) (width 0.4) (layer "B.Cu") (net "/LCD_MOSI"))
 (segment (start 67.39 95.67) (end 67.39 96.72) (width 0.4) (layer "B.Cu") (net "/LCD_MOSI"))
 (segment (start 88 106.539999) (end 83.6 106.539999) (width 0.8) (layer "F.Cu") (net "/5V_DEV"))
 (segment (start 83.6 106.539999) (end 83.6 97.72) (width 0.8) (layer "F.Cu") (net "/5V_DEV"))
 (segment (start 141.5 107) (end 128 107) (width 0.8) (layer "F.Cu") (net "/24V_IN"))
 (segment (start 132.62 95.539999) (end 141.5 96.84) (width 0.6) (layer "F.Cu") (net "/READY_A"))
 (segment (start 132.62 93) (end 141.5 91.759999) (width 0.6) (layer "F.Cu") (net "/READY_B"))
 (segment (start 132.62 85.44) (end 141.5 86.68) (width 0.6) (layer "F.Cu") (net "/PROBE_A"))
 (segment (start 132.62 82.9) (end 141.5 81.6) (width 0.6) (layer "F.Cu") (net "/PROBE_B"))
 (segment (start 128 101.92) (end 125 101.92) (width 0.8) (layer "B.Cu") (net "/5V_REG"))
 (segment (start 122.92 104) (end 88 104) (width 0.8) (layer "B.Cu") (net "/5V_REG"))
 (segment (start 125 101.92) (end 122.92 104) (width 0.8) (layer "B.Cu") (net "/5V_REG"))
 (segment (start 121.62 93) (end 125 93) (width 0.4) (layer "F.Cu") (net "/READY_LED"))
 (segment (start 121.62 82.9) (end 125 82.9) (width 0.4) (layer "F.Cu") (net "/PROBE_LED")))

